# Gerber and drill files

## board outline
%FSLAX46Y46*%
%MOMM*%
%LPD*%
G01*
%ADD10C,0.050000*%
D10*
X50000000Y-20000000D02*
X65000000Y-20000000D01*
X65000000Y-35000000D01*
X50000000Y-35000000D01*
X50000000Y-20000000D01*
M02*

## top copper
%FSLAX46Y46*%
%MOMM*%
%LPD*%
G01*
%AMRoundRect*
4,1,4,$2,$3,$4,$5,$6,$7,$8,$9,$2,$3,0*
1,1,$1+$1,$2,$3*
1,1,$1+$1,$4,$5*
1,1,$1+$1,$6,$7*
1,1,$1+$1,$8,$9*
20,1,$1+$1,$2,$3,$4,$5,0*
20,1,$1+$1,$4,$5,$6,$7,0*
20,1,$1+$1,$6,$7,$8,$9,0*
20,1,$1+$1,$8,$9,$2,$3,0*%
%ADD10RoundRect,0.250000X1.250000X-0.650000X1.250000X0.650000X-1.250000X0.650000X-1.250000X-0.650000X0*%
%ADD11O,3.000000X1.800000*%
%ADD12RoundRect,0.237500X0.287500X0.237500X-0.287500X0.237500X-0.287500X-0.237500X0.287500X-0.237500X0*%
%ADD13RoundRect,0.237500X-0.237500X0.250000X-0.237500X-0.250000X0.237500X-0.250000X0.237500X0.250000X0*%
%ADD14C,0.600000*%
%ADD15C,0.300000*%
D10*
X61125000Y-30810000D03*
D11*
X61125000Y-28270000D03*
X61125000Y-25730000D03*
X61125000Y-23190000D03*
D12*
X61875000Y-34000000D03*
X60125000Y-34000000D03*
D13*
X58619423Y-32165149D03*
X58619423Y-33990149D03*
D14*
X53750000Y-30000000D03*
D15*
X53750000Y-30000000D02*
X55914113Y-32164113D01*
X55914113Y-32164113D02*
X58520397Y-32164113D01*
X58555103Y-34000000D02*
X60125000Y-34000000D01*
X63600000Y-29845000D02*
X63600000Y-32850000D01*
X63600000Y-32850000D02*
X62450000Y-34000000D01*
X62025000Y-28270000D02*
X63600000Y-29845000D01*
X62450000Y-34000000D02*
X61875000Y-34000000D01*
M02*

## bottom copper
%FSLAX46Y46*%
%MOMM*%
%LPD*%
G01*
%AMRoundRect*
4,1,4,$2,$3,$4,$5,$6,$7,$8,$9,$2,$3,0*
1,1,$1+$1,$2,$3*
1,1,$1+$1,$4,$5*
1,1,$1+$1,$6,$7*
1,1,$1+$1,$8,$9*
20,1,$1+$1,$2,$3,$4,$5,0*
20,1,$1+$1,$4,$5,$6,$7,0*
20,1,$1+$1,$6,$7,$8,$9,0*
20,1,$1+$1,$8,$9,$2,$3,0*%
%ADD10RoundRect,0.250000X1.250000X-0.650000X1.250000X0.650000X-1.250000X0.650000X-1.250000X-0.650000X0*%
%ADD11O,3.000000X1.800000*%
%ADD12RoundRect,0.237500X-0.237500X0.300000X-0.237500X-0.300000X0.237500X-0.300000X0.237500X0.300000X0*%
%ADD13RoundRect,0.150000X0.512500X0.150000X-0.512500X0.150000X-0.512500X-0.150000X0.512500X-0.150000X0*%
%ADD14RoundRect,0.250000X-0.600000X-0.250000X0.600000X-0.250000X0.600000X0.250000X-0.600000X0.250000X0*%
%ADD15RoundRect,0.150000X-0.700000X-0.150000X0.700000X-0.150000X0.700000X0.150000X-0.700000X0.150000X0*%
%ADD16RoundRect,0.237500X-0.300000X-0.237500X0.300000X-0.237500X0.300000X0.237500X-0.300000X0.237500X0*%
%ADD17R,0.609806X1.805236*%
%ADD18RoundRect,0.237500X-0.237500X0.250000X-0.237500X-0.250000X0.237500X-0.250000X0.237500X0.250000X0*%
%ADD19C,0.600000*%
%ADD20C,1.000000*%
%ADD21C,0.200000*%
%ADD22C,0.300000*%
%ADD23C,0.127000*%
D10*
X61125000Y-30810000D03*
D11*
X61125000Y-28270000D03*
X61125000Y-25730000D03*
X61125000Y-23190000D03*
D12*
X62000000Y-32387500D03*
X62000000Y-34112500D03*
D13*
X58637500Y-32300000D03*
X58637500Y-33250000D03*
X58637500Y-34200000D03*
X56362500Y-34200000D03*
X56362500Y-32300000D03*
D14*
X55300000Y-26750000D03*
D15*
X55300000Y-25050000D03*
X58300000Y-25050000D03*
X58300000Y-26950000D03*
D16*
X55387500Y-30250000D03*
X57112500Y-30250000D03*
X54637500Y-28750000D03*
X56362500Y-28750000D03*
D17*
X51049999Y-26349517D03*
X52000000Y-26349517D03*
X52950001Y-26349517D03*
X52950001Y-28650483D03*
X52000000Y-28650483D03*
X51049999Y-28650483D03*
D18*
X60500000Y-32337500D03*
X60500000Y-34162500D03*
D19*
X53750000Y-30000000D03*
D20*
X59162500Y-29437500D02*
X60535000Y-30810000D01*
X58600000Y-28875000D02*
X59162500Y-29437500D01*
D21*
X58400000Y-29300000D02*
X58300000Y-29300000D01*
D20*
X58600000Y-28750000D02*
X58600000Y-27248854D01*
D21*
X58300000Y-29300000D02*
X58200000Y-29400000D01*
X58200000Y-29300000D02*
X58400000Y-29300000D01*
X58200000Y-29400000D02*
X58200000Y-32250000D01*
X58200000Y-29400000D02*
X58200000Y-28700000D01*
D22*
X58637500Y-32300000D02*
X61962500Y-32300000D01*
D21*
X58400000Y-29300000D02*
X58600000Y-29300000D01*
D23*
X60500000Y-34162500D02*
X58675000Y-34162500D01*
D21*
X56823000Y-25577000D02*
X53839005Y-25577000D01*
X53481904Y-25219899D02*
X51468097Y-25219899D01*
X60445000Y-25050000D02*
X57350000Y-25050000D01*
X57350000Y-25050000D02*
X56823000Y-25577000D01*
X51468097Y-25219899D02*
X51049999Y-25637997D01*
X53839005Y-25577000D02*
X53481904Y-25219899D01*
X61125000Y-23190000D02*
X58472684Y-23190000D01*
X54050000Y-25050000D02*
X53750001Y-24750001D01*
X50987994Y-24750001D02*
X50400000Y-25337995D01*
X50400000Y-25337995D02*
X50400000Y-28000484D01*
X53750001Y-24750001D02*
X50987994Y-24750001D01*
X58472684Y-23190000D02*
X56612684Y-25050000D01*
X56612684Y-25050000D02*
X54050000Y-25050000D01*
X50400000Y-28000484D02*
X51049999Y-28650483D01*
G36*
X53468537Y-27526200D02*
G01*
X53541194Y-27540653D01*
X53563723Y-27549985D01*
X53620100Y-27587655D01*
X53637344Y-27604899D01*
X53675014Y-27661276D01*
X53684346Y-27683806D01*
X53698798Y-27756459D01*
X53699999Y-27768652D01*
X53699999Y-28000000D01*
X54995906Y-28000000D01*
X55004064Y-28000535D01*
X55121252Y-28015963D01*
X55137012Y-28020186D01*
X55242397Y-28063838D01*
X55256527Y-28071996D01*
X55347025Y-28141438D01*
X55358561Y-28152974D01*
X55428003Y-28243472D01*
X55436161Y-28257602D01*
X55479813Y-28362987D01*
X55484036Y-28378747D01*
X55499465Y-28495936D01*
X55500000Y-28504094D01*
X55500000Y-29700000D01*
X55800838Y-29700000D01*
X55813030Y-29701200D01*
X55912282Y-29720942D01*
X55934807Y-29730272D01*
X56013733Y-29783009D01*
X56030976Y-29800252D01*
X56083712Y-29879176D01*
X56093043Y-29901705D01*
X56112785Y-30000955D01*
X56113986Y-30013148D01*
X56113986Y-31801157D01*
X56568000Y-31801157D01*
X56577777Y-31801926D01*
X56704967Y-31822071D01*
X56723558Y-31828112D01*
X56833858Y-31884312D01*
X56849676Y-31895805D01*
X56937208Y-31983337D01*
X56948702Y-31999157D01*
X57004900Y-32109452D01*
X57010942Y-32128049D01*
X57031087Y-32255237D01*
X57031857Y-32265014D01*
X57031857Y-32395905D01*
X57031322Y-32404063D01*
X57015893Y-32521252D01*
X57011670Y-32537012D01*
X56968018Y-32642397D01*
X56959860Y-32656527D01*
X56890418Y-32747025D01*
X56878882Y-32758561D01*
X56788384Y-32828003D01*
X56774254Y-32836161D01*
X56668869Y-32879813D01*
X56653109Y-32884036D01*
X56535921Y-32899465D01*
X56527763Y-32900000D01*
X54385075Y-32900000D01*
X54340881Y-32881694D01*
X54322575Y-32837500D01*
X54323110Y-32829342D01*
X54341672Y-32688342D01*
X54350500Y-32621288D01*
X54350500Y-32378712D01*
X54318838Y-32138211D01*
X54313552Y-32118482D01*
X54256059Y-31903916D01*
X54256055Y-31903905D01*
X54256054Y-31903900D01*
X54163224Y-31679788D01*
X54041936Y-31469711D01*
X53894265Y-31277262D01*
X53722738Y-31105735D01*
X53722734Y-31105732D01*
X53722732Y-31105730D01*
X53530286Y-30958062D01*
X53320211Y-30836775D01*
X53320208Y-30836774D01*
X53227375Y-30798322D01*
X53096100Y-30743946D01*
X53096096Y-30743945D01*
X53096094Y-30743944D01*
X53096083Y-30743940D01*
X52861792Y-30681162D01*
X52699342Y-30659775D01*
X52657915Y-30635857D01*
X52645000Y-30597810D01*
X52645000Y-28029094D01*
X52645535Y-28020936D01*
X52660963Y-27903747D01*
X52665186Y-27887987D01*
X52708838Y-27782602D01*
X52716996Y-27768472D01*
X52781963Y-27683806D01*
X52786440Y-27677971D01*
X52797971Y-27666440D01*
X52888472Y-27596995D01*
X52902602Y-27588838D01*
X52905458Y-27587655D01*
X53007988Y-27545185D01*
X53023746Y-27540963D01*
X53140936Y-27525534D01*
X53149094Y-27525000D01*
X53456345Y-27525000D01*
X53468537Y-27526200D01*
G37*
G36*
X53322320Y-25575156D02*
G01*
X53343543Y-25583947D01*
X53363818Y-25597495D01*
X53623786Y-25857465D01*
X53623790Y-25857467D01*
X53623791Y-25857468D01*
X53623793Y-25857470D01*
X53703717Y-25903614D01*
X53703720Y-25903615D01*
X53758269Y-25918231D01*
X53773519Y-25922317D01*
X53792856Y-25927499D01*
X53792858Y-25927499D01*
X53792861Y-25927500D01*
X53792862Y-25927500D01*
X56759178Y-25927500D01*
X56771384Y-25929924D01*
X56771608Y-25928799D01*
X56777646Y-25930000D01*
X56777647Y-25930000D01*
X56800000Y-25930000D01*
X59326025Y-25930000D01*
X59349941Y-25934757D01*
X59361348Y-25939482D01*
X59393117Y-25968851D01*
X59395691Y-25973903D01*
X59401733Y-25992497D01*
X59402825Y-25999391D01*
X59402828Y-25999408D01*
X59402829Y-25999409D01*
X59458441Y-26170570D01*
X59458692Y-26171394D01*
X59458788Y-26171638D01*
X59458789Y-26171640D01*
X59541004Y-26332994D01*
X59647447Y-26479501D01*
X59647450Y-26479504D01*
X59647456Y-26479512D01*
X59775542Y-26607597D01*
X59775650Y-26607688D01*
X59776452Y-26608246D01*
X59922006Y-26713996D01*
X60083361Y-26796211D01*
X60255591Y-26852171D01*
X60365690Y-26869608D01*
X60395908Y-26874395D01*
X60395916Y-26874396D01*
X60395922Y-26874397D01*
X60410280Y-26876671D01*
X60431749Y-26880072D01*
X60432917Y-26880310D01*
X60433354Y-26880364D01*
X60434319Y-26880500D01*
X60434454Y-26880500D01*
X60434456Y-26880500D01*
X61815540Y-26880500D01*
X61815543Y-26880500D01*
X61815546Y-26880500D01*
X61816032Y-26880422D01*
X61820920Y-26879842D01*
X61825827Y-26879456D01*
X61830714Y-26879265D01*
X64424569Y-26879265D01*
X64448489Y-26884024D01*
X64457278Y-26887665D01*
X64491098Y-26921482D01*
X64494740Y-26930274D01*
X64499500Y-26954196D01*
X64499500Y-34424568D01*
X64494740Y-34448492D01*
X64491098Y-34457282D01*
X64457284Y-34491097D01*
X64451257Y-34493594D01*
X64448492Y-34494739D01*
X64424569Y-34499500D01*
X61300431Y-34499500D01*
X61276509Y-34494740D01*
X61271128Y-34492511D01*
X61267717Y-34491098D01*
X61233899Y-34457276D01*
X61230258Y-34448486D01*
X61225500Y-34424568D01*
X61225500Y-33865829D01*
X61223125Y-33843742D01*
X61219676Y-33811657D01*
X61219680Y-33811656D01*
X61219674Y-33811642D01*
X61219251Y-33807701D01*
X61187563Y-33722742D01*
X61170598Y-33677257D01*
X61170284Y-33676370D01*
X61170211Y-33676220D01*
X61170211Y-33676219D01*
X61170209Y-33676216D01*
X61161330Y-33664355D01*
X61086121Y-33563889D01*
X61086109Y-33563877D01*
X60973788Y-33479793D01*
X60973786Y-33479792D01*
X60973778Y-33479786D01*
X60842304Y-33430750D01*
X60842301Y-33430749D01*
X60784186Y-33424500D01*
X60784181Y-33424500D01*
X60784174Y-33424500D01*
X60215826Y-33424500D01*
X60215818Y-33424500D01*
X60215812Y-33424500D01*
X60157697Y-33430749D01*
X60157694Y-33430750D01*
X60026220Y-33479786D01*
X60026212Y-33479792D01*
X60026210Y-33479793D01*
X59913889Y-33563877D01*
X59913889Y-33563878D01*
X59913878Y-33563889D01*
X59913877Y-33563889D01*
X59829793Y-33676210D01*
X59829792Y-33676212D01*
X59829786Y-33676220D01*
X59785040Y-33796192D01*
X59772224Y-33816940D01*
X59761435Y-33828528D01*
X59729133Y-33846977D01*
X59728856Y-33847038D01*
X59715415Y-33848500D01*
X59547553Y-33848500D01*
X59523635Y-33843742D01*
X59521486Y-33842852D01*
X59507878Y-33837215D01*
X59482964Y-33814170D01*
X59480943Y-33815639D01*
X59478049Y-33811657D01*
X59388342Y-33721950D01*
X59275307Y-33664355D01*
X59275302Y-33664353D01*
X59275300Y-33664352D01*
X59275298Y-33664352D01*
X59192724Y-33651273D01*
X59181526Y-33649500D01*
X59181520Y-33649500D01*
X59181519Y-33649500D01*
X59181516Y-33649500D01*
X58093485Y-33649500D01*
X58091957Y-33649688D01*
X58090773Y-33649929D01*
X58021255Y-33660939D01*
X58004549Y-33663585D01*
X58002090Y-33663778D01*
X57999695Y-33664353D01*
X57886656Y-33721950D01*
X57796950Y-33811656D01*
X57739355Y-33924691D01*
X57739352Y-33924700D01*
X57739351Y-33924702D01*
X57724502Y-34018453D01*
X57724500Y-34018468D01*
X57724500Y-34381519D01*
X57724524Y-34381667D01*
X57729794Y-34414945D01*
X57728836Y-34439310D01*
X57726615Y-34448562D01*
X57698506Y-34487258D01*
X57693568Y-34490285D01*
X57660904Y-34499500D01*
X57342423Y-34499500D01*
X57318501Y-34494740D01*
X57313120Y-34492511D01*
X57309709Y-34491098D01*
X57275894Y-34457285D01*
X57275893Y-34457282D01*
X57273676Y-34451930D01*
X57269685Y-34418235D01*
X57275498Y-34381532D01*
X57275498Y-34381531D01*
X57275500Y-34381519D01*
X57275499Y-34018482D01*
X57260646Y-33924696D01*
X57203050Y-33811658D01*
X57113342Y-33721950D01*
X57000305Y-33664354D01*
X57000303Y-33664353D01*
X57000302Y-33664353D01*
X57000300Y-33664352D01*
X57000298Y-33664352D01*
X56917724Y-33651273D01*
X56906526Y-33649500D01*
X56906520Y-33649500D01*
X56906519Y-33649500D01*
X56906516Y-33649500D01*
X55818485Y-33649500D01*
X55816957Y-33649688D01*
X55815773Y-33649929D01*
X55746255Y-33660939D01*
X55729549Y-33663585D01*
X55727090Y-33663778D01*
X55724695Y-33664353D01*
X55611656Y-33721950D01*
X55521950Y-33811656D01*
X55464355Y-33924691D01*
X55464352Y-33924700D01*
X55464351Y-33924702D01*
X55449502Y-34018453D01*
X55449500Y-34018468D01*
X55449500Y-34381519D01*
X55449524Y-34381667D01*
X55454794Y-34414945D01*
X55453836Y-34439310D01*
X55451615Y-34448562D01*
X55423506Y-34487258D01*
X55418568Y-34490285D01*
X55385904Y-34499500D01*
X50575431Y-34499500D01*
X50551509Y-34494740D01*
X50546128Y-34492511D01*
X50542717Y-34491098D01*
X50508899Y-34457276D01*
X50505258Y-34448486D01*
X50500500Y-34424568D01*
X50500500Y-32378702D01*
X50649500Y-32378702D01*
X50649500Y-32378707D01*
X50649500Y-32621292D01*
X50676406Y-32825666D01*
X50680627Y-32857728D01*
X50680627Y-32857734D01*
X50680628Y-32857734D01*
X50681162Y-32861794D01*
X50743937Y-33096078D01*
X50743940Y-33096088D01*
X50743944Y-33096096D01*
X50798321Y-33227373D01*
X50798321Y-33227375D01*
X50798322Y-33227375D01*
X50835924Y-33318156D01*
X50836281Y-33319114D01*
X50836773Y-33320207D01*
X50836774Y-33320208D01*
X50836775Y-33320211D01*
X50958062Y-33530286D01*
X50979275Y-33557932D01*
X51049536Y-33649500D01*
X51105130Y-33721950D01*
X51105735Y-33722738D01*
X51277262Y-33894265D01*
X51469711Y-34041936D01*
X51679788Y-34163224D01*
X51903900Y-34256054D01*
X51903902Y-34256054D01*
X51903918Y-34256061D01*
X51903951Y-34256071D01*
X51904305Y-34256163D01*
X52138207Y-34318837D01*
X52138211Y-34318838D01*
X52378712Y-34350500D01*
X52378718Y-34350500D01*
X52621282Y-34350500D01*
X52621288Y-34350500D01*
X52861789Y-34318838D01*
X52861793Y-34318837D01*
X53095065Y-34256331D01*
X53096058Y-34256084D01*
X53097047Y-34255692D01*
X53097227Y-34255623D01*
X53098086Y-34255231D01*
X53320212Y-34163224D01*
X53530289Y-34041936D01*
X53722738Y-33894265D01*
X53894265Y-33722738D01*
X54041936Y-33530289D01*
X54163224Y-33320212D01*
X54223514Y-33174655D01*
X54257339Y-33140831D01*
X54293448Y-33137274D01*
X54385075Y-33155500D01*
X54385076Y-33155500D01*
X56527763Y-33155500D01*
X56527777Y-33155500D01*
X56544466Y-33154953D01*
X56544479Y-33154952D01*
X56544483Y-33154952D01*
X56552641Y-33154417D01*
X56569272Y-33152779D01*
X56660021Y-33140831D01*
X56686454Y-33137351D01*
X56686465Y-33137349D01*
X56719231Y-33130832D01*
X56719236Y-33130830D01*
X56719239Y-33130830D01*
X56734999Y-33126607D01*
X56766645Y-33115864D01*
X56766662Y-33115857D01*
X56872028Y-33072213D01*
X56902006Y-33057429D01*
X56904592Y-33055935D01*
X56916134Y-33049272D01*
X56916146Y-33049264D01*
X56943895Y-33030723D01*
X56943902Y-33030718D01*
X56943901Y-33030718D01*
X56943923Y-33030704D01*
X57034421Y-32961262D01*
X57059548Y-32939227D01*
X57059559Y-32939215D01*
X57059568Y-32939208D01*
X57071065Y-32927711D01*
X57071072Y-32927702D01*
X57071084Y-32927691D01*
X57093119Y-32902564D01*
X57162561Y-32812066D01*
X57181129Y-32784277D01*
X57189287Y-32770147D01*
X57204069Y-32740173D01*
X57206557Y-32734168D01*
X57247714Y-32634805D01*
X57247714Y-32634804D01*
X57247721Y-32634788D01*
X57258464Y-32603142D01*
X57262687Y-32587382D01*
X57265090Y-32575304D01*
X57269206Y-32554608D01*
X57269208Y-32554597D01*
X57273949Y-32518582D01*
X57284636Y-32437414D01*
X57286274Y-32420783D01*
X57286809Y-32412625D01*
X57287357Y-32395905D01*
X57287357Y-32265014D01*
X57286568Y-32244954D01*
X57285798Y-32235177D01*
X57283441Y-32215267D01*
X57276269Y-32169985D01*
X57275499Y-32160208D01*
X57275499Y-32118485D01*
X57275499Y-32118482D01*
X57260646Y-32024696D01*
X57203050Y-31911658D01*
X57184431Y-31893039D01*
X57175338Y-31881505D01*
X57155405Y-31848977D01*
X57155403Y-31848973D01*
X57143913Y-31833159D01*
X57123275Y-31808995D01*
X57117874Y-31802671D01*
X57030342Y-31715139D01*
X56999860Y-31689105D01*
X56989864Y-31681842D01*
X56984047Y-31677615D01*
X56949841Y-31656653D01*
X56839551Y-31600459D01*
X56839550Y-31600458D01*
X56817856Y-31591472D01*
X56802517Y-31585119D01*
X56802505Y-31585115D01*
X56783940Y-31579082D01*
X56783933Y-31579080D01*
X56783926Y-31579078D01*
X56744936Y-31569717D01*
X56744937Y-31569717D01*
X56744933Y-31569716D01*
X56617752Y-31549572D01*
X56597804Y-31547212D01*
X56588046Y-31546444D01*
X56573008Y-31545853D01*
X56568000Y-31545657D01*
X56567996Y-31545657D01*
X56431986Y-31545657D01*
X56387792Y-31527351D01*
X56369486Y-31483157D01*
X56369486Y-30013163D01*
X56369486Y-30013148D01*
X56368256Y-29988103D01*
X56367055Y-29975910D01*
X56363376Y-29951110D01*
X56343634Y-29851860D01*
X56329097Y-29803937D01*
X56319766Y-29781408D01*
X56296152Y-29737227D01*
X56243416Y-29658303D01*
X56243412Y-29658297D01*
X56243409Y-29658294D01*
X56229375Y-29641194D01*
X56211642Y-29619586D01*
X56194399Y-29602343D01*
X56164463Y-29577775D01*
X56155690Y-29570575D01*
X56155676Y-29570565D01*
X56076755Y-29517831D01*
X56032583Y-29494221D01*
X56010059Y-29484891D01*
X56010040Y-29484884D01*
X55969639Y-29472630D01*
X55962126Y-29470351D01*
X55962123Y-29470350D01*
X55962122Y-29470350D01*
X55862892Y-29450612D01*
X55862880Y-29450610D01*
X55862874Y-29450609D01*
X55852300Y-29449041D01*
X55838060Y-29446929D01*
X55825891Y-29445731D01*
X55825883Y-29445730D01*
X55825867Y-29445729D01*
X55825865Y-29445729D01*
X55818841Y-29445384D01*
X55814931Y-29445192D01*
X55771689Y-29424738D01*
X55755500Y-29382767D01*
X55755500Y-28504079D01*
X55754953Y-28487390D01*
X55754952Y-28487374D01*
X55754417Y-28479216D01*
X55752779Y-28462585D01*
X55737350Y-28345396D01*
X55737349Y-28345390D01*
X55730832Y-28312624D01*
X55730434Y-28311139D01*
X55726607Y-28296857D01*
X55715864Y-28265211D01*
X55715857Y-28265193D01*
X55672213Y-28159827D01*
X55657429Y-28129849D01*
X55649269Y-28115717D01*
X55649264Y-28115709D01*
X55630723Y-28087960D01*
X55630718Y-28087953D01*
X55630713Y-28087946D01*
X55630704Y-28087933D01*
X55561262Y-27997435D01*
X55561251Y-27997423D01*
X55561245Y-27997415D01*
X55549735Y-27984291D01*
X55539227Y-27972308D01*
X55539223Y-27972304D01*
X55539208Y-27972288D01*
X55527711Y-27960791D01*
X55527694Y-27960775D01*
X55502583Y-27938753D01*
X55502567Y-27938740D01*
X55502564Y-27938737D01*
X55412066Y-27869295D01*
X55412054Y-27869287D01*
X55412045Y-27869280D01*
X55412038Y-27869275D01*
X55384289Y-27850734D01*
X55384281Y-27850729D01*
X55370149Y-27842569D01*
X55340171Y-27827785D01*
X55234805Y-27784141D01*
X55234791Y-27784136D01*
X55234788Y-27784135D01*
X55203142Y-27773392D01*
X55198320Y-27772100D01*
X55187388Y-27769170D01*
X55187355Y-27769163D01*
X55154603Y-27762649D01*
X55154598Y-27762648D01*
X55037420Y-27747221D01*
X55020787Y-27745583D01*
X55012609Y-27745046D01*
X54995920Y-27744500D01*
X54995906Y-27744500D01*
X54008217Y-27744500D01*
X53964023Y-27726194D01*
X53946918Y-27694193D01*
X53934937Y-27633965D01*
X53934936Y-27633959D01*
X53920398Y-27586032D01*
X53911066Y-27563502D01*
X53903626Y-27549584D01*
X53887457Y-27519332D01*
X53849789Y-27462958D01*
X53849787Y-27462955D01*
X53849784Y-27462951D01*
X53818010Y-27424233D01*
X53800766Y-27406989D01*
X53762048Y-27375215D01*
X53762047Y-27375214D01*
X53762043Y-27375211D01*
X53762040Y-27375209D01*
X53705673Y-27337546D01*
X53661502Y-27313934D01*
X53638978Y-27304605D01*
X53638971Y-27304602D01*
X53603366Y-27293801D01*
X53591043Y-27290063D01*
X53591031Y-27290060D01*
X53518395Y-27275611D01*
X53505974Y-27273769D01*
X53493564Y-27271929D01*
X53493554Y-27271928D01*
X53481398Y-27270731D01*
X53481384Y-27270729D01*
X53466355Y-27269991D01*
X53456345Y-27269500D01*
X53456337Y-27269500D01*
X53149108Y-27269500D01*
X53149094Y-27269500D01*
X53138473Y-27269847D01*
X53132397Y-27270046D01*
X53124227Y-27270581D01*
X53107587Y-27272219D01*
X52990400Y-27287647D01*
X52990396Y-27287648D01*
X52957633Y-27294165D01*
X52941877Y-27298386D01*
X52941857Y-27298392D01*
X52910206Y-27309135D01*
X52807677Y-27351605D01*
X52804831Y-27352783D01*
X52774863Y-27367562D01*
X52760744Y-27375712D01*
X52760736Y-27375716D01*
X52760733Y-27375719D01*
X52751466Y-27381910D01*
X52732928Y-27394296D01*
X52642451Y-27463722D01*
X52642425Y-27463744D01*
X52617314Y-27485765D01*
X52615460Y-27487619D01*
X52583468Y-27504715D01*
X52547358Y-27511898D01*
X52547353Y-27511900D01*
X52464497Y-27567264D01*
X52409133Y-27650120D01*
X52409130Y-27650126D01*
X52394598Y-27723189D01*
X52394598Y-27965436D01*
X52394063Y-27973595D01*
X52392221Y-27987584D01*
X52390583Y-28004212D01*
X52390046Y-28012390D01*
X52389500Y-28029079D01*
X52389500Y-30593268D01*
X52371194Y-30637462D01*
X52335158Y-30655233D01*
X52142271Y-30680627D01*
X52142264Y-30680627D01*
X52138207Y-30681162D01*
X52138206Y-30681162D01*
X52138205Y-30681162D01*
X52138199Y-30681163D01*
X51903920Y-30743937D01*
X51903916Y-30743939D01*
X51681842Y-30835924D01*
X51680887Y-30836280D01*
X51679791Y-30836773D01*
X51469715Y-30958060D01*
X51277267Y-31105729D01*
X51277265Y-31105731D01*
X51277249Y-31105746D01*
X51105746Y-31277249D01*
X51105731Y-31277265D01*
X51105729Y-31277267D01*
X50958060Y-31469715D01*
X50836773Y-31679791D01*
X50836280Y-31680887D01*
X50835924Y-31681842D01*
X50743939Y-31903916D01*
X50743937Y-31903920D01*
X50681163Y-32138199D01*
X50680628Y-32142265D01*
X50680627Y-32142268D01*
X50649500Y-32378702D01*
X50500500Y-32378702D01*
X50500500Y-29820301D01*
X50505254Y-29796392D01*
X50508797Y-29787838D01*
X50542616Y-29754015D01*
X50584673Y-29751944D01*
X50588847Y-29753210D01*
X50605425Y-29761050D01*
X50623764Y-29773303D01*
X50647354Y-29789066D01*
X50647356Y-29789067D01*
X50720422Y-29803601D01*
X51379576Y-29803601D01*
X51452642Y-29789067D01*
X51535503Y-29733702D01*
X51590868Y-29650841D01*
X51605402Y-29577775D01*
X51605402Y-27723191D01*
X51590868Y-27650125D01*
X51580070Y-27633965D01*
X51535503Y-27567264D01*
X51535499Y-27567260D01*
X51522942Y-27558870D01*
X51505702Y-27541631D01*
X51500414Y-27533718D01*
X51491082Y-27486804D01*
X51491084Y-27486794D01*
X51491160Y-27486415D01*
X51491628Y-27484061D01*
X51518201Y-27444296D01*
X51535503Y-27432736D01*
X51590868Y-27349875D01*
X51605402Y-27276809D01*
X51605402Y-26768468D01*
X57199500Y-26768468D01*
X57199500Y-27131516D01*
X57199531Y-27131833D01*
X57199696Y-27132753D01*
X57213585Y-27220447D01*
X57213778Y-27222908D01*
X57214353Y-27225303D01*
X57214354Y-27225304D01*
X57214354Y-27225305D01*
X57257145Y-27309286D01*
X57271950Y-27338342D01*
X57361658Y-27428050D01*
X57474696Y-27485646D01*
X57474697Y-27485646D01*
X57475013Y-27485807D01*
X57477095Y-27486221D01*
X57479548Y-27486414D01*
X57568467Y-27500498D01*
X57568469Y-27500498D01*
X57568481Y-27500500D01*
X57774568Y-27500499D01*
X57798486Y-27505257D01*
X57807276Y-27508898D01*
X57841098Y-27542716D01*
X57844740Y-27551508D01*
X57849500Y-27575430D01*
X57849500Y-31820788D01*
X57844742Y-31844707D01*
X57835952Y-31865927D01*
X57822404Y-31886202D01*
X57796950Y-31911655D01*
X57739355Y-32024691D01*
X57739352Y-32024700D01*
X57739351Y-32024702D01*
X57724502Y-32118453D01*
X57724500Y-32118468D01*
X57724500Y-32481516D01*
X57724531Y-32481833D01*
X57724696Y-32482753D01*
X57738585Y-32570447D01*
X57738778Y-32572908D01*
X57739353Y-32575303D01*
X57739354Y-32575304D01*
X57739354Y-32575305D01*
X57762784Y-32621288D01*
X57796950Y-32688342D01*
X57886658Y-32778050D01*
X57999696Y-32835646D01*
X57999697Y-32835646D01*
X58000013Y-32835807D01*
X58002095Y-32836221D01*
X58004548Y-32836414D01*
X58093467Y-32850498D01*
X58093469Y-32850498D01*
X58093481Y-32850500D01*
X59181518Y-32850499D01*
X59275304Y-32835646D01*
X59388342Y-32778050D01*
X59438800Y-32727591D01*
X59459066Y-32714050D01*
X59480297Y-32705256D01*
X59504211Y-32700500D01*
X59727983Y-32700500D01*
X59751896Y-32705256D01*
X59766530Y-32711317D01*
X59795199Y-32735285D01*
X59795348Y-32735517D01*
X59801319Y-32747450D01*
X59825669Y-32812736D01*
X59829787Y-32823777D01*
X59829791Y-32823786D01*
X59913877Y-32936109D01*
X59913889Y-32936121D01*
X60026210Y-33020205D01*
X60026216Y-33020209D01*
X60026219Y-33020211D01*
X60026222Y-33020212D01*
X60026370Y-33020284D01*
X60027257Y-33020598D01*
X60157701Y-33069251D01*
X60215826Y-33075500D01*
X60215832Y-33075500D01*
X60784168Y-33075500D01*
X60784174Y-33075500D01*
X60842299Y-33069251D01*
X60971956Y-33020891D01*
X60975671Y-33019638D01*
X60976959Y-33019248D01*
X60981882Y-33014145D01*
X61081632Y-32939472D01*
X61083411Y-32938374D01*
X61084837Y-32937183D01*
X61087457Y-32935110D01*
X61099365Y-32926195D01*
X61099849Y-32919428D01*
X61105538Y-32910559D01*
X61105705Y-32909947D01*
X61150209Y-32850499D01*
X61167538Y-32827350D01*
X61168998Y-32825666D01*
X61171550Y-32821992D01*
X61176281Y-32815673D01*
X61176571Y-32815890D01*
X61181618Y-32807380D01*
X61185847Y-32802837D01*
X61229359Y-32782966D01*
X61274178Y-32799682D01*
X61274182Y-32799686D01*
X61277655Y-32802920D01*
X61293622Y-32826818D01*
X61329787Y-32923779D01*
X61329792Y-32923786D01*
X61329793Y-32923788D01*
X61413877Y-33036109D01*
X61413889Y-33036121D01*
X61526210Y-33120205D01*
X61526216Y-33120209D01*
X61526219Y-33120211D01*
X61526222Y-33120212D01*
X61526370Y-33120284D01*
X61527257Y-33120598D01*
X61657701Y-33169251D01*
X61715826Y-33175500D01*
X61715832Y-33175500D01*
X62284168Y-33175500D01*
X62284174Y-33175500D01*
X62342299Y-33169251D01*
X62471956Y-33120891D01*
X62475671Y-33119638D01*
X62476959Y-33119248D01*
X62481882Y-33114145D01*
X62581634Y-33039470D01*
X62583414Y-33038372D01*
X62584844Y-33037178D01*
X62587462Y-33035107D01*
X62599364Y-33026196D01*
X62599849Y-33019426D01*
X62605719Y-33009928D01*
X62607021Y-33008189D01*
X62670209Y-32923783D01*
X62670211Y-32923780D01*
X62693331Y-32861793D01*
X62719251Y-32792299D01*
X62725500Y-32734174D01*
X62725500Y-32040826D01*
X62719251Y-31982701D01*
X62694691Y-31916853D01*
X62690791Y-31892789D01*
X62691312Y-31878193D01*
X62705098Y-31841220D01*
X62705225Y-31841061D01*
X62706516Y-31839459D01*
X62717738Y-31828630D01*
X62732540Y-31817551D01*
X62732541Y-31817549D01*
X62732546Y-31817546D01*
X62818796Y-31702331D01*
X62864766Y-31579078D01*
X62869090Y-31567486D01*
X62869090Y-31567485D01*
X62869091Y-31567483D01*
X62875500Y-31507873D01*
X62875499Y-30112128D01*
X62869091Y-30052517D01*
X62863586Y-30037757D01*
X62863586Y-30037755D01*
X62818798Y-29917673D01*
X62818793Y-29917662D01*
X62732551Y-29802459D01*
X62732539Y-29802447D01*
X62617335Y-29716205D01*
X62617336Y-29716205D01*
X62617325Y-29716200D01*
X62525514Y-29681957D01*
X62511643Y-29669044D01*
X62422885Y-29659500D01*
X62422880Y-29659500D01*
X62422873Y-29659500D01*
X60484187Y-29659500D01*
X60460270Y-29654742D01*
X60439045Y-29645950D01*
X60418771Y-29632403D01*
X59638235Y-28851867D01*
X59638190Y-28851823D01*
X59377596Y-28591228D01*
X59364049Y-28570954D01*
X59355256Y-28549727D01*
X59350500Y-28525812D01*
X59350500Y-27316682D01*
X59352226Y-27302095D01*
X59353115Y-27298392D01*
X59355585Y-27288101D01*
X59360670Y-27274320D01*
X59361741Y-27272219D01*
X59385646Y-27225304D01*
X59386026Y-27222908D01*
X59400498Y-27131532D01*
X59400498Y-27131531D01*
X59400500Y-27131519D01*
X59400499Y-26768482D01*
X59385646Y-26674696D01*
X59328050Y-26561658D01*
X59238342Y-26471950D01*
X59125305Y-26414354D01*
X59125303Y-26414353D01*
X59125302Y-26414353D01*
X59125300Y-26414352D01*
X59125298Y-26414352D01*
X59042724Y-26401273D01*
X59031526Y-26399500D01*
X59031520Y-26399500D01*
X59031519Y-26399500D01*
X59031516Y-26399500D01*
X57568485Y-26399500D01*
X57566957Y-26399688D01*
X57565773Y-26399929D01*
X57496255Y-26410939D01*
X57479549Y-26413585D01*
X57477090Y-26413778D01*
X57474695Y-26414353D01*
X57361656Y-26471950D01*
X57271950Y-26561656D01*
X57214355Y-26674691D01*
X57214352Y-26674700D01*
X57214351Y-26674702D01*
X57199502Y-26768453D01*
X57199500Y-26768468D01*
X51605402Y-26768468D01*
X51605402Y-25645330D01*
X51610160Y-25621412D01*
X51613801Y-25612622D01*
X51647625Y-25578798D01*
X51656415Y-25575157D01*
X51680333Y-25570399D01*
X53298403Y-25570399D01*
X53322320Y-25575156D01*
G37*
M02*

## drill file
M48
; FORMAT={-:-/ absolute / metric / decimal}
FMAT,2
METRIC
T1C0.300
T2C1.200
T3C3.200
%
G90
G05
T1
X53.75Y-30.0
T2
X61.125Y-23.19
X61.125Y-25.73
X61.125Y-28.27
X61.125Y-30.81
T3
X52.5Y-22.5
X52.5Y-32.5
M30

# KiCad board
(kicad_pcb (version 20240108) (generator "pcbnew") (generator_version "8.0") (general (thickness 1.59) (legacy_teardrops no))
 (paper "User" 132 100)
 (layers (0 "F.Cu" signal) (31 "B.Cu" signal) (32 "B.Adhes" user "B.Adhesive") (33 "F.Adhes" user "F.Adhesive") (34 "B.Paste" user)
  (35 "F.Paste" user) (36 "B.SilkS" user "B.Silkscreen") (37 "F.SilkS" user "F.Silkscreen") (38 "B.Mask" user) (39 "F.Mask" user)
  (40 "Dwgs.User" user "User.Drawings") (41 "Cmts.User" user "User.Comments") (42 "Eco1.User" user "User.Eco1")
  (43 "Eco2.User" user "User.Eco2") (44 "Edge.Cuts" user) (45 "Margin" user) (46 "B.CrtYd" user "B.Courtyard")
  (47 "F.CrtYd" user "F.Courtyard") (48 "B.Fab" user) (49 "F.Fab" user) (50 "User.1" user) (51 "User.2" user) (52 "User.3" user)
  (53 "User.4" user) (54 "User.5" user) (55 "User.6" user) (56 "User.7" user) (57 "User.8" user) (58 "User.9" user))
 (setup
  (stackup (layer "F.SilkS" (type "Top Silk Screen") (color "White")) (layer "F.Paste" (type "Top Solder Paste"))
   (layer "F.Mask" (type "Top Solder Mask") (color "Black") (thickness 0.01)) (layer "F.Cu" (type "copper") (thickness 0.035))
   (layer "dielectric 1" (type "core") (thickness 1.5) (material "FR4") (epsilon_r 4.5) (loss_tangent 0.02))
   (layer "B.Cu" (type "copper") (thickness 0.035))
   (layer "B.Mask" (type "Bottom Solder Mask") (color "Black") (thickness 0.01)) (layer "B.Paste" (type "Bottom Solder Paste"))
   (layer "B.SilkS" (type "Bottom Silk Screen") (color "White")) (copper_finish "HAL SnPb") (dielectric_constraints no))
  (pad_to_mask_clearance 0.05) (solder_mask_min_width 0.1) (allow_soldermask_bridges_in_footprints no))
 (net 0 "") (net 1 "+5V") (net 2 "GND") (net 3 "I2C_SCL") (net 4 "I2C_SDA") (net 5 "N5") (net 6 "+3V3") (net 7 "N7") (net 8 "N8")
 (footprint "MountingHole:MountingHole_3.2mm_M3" (layer "F.Cu") (at 52.5 22.5)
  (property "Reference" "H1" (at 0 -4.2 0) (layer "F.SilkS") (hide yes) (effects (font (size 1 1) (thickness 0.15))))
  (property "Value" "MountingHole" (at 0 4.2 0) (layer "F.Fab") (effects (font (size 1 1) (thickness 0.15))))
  (pad "" np_thru_hole circle (at 0 0) (size 3.2 3.2) (drill 3.2) (layers "*.Cu" "*.Mask")))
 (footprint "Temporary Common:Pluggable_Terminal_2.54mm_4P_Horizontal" (layer "F.Cu") (at 57.675 26.78 90)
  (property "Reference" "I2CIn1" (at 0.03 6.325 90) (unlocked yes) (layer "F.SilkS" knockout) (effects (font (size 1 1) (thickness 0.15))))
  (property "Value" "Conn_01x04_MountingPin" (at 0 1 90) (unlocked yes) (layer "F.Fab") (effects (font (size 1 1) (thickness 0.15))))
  (pad "1" thru_hole roundrect (at -4.03 3.45 90) (size 1.8 3) (drill 1.2) (layers "*.Cu" "*.Mask") (remove_unused_layers no)
   (roundrect_rratio 0.138889) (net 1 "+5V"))
  (pad "2" thru_hole oval (at -1.49 3.45 90) (size 1.8 3) (drill 1.2) (layers "*.Cu" "*.Mask") (remove_unused_layers no) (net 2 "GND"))
  (pad "3" thru_hole oval (at 1.05 3.45 90) (size 1.8 3) (drill 1.2) (layers "*.Cu" "*.Mask") (remove_unused_layers no) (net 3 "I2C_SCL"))
  (pad "4" thru_hole oval (at 3.59 3.45 90) (size 1.8 3) (drill 1.2) (layers "*.Cu" "*.Mask") (remove_unused_layers no) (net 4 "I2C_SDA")))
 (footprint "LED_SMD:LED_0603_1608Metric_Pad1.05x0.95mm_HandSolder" (layer "F.Cu") (at 61 34 180)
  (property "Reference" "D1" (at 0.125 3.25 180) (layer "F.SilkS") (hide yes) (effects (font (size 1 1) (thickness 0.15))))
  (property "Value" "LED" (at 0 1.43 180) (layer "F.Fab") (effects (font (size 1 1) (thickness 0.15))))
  (pad "1" smd roundrect (at -0.875 0 180) (size 1.05 0.95) (layers "F.Cu" "F.Paste" "F.Mask") (roundrect_rratio 0.25) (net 2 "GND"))
  (pad "2" smd roundrect (at 0.875 0 180) (size 1.05 0.95) (layers "F.Cu" "F.Paste" "F.Mask") (roundrect_rratio 0.25) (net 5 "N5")))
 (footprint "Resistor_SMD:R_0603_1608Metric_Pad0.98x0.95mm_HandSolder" (layer "F.Cu") (at 58.619423 33.077649 -90)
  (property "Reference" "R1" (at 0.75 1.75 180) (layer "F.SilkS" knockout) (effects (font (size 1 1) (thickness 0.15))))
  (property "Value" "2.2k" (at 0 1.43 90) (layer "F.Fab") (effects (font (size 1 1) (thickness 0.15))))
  (pad "1" smd roundrect (at -0.9125 0 270) (size 0.975 0.95) (layers "F.Cu" "F.Paste" "F.Mask") (roundrect_rratio 0.25) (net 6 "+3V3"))
  (pad "2" smd roundrect (at 0.9125 0 270) (size 0.975 0.95) (layers "F.Cu" "F.Paste" "F.Mask") (roundrect_rratio 0.25) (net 5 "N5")))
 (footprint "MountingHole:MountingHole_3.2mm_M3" (layer "F.Cu") (at 52.5 32.5)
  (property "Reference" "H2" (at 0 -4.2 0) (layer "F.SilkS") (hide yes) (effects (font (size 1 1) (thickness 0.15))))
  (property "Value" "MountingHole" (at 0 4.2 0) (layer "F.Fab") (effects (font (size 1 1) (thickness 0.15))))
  (pad "" np_thru_hole circle (at 0 0) (size 3.2 3.2) (drill 3.2) (layers "*.Cu" "*.Mask")))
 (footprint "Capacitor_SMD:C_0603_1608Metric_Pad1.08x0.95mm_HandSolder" (layer "B.Cu") (at 62 33.25 -90)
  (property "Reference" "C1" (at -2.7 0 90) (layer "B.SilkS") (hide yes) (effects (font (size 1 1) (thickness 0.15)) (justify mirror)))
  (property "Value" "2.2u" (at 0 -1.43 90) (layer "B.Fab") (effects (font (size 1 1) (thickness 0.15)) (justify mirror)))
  (pad "1" smd roundrect (at -0.8625 0 270) (size 1.075 0.95) (layers "B.Cu" "B.Paste" "B.Mask") (roundrect_rratio 0.25) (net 1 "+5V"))
  (pad "2" smd roundrect (at 0.8625 0 270) (size 1.075 0.95) (layers "B.Cu" "B.Paste" "B.Mask") (roundrect_rratio 0.25) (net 2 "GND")))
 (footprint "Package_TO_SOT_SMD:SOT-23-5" (layer "B.Cu") (at 57.5 33.25 180)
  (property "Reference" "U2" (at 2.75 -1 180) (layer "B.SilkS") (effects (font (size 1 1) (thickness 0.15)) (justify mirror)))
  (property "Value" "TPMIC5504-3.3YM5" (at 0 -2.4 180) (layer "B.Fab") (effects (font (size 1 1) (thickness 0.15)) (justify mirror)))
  (pad "1" smd roundrect (at -1.1375 0.95 180) (size 1.325 0.6) (layers "B.Cu" "B.Paste" "B.Mask") (roundrect_rratio 0.25) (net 1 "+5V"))
  (pad "2" smd roundrect (at -1.1375 0 180) (size 1.325 0.6) (layers "B.Cu" "B.Paste" "B.Mask") (roundrect_rratio 0.25) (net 2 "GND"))
  (pad "3" smd roundrect (at -1.1375 -0.95 180) (size 1.325 0.6) (layers "B.Cu" "B.Paste" "B.Mask") (roundrect_rratio 0.25) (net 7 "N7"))
  (pad "4" smd roundrect (at 1.1375 -0.95 180) (size 1.325 0.6) (layers "B.Cu" "B.Paste" "B.Mask") (roundrect_rratio 0.25) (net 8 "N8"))
  (pad "5" smd roundrect (at 1.1375 0.95 180) (size 1.325 0.6) (layers "B.Cu" "B.Paste" "B.Mask") (roundrect_rratio 0.25) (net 6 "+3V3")))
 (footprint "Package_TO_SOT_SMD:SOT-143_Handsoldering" (layer "B.Cu") (at 56.8 26)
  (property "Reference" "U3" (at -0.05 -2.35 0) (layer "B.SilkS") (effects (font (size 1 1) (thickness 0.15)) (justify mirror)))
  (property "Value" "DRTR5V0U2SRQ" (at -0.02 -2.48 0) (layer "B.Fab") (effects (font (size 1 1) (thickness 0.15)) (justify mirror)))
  (pad "1" smd roundrect (at -1.5 0.75) (size 1.7 1) (layers "B.Cu" "B.Paste" "B.Mask") (roundrect_rratio 0.25) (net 2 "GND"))
  (pad "2" smd roundrect (at -1.5 -0.95) (size 1.7 0.6) (layers "B.Cu" "B.Paste" "B.Mask") (roundrect_rratio 0.25) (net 4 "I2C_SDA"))
  (pad "3" smd roundrect (at 1.5 -0.95) (size 1.7 0.6) (layers "B.Cu" "B.Paste" "B.Mask") (roundrect_rratio 0.25) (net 3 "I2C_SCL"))
  (pad "4" smd roundrect (at 1.5 0.95) (size 1.7 0.6) (layers "B.Cu" "B.Paste" "B.Mask") (roundrect_rratio 0.25) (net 1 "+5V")))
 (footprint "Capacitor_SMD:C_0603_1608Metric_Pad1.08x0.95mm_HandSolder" (layer "B.Cu") (at 56.25 30.25)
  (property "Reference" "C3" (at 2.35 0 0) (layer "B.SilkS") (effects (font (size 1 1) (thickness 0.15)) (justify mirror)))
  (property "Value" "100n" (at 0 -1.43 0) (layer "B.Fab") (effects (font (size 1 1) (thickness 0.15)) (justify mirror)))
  (pad "1" smd roundrect (at -0.8625 0) (size 1.075 0.95) (layers "B.Cu" "B.Paste" "B.Mask") (roundrect_rratio 0.25) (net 6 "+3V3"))
  (pad "2" smd roundrect (at 0.8625 0) (size 1.075 0.95) (layers "B.Cu" "B.Paste" "B.Mask") (roundrect_rratio 0.25) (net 2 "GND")))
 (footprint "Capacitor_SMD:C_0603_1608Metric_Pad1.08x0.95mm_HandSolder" (layer "B.Cu") (at 55.5 28.75)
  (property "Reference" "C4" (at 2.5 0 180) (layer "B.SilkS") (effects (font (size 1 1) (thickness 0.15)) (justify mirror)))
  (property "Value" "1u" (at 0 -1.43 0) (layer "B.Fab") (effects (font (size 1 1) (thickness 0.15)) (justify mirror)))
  (pad "1" smd roundrect (at -0.8625 0) (size 1.075 0.95) (layers "B.Cu" "B.Paste" "B.Mask") (roundrect_rratio 0.25) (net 6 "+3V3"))
  (pad "2" smd roundrect (at 0.8625 0) (size 1.075 0.95) (layers "B.Cu" "B.Paste" "B.Mask") (roundrect_rratio 0.25) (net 2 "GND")))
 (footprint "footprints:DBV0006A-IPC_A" (layer "B.Cu") (at 52 27.5 -90)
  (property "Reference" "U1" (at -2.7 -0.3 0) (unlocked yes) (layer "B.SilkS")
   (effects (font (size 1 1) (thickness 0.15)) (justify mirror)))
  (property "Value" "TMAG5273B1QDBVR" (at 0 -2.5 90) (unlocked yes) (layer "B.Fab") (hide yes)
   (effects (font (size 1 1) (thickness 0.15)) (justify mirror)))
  (pad "1" smd rect (at -1.150483 0.950001 270) (size 1.805236 0.609806) (layers "B.Cu" "B.Paste" "B.Mask") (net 3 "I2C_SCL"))
  (pad "2" smd rect (at -1.150483 0 270) (size 1.805236 0.609806) (layers "B.Cu" "B.Paste" "B.Mask") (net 2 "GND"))
  (pad "3" smd rect (at -1.150483 -0.950001 270) (size 1.805236 0.609806) (layers "B.Cu" "B.Paste" "B.Mask") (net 2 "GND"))
  (pad "4" smd rect (at 1.150483 -0.950001 270) (size 1.805236 0.609806) (layers "B.Cu" "B.Paste" "B.Mask") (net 6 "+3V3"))
  (pad "5" smd rect (at 1.150483 0 270) (size 1.805236 0.609806) (layers "B.Cu" "B.Paste" "B.Mask") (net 2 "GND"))
  (pad "6" smd rect (at 1.150483 0.950001 270) (size 1.805236 0.609806) (layers "B.Cu" "B.Paste" "B.Mask") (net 4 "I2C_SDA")))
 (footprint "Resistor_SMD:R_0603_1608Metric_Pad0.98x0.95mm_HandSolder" (layer "B.Cu") (at 60.5 33.25 -90)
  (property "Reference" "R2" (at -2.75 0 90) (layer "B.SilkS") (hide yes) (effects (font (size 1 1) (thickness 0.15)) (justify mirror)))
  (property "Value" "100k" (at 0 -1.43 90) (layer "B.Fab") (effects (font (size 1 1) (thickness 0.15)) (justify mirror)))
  (pad "1" smd roundrect (at -0.9125 0 270) (size 0.975 0.95) (layers "B.Cu" "B.Paste" "B.Mask") (roundrect_rratio 0.25) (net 1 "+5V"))
  (pad "2" smd roundrect (at 0.9125 0 270) (size 0.975 0.95) (layers "B.Cu" "B.Paste" "B.Mask") (roundrect_rratio 0.25) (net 7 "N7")))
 (gr_rect (start 50 20) (end 65 35) (stroke (width 0.05) (type default)) (fill none) (layer "Edge.Cuts"))
 (segment (start 59.1625 29.4375) (end 60.535 30.81) (width 1) (layer "B.Cu") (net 1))
 (segment (start 58.6 28.875) (end 59.1625 29.4375) (width 1) (layer "B.Cu") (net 1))
 (segment (start 58.4 29.3) (end 58.3 29.3) (width 0.2) (layer "B.Cu") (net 1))
 (segment (start 58.6 28.75) (end 58.6 27.248854) (width 1) (layer "B.Cu") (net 1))
 (segment (start 58.3 29.3) (end 58.2 29.4) (width 0.2) (layer "B.Cu") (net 1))
 (segment (start 58.2 29.3) (end 58.4 29.3) (width 0.2) (layer "B.Cu") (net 1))
 (segment (start 58.2 29.4) (end 58.2 32.25) (width 0.2) (layer "B.Cu") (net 1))
 (segment (start 58.2 29.4) (end 58.2 28.7) (width 0.2) (layer "B.Cu") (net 1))
 (segment (start 58.6375 32.3) (end 61.9625 32.3) (width 0.3) (layer "B.Cu") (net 1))
 (segment (start 58.4 29.3) (end 58.6 29.3) (width 0.2) (layer "B.Cu") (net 1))
 (segment (start 60.5 34.1625) (end 58.675 34.1625) (width 0.127) (layer "B.Cu") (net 7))
 (segment (start 53.75 30) (end 55.914113 32.164113) (width 0.3) (layer "F.Cu") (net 6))
 (segment (start 55.914113 32.164113) (end 58.520397 32.164113) (width 0.3) (layer "F.Cu") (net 6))
 (via (at 53.75 30) (size 0.6) (drill 0.3) (layers "F.Cu" "B.Cu") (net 6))
 (segment (start 58.555103 34) (end 60.125 34) (width 0.3) (layer "F.Cu") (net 5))
 (segment (start 56.823 25.577) (end 53.839005 25.577) (width 0.2) (layer "B.Cu") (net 3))
 (segment (start 53.481904 25.219899) (end 51.468097 25.219899) (width 0.2) (layer "B.Cu") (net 3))
 (segment (start 60.445 25.05) (end 57.35 25.05) (width 0.2) (layer "B.Cu") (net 3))
 (segment (start 57.35 25.05) (end 56.823 25.577) (width 0.2) (layer "B.Cu") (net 3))
 (segment (start 51.468097 25.219899) (end 51.049999 25.637997) (width 0.2) (layer "B.Cu") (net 3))
 (segment (start 53.839005 25.577) (end 53.481904 25.219899) (width 0.2) (layer "B.Cu") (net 3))
 (segment (start 61.125 23.19) (end 58.472684 23.19) (width 0.2) (layer "B.Cu") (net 4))
 (segment (start 54.05 25.05) (end 53.750001 24.750001) (width 0.2) (layer "B.Cu") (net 4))
 (segment (start 50.987994 24.750001) (end 50.4 25.337995) (width 0.2) (layer "B.Cu") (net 4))
 (segment (start 50.4 25.337995) (end 50.4 28.000484) (width 0.2) (layer "B.Cu") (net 4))
 (segment (start 53.750001 24.750001) (end 50.987994 24.750001) (width 0.2) (layer "B.Cu") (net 4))
 (segment (start 58.472684 23.19) (end 56.612684 25.05) (width 0.2) (layer "B.Cu") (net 4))
 (segment (start 56.612684 25.05) (end 54.05 25.05) (width 0.2) (layer "B.Cu") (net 4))
 (segment (start 50.4 28.000484) (end 51.049999 28.650483) (width 0.2) (layer "B.Cu") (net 4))
 (segment (start 63.6 29.845) (end 63.6 32.85) (width 0.3) (layer "F.Cu") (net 2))
 (segment (start 63.6 32.85) (end 62.45 34) (width 0.3) (layer "F.Cu") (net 2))
 (segment (start 62.025 28.27) (end 63.6 29.845) (width 0.3) (layer "F.Cu") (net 2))
 (segment (start 62.45 34) (end 61.875 34) (width 0.3) (layer "F.Cu") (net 2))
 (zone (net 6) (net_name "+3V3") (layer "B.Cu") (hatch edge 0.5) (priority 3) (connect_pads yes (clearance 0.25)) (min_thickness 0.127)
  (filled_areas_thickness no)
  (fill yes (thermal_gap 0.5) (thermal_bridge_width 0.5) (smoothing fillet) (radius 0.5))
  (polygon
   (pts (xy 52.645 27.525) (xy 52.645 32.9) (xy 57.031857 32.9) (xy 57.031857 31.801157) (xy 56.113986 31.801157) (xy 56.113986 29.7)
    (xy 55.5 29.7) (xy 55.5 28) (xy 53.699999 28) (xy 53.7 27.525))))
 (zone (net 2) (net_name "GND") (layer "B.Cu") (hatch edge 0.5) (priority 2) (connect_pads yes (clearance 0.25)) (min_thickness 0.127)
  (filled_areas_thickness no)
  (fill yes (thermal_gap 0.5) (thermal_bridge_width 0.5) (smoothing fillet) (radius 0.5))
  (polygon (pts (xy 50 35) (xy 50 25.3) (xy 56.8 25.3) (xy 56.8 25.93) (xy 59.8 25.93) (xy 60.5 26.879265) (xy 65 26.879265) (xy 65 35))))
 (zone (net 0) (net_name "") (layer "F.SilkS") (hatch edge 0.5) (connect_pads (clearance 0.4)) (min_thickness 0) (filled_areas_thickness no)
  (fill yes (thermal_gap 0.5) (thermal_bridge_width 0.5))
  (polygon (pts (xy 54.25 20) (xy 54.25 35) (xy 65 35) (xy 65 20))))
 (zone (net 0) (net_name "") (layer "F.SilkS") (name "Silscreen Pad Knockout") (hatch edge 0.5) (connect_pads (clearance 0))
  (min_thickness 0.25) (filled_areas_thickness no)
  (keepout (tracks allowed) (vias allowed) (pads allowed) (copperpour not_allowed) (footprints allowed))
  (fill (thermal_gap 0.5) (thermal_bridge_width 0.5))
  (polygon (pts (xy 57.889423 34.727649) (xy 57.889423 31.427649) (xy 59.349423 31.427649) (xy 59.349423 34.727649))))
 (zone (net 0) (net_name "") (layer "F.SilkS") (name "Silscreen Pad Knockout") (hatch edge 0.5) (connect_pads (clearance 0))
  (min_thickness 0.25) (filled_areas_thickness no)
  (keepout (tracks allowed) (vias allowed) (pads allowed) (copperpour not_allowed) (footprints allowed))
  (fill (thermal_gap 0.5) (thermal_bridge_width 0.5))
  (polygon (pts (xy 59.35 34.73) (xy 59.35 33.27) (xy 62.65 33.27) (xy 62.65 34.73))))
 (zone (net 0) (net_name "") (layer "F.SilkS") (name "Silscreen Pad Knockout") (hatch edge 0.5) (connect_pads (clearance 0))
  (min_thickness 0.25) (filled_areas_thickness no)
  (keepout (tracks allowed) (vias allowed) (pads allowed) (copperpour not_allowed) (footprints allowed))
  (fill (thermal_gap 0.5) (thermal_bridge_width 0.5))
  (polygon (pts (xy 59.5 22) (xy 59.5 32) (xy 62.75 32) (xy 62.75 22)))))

